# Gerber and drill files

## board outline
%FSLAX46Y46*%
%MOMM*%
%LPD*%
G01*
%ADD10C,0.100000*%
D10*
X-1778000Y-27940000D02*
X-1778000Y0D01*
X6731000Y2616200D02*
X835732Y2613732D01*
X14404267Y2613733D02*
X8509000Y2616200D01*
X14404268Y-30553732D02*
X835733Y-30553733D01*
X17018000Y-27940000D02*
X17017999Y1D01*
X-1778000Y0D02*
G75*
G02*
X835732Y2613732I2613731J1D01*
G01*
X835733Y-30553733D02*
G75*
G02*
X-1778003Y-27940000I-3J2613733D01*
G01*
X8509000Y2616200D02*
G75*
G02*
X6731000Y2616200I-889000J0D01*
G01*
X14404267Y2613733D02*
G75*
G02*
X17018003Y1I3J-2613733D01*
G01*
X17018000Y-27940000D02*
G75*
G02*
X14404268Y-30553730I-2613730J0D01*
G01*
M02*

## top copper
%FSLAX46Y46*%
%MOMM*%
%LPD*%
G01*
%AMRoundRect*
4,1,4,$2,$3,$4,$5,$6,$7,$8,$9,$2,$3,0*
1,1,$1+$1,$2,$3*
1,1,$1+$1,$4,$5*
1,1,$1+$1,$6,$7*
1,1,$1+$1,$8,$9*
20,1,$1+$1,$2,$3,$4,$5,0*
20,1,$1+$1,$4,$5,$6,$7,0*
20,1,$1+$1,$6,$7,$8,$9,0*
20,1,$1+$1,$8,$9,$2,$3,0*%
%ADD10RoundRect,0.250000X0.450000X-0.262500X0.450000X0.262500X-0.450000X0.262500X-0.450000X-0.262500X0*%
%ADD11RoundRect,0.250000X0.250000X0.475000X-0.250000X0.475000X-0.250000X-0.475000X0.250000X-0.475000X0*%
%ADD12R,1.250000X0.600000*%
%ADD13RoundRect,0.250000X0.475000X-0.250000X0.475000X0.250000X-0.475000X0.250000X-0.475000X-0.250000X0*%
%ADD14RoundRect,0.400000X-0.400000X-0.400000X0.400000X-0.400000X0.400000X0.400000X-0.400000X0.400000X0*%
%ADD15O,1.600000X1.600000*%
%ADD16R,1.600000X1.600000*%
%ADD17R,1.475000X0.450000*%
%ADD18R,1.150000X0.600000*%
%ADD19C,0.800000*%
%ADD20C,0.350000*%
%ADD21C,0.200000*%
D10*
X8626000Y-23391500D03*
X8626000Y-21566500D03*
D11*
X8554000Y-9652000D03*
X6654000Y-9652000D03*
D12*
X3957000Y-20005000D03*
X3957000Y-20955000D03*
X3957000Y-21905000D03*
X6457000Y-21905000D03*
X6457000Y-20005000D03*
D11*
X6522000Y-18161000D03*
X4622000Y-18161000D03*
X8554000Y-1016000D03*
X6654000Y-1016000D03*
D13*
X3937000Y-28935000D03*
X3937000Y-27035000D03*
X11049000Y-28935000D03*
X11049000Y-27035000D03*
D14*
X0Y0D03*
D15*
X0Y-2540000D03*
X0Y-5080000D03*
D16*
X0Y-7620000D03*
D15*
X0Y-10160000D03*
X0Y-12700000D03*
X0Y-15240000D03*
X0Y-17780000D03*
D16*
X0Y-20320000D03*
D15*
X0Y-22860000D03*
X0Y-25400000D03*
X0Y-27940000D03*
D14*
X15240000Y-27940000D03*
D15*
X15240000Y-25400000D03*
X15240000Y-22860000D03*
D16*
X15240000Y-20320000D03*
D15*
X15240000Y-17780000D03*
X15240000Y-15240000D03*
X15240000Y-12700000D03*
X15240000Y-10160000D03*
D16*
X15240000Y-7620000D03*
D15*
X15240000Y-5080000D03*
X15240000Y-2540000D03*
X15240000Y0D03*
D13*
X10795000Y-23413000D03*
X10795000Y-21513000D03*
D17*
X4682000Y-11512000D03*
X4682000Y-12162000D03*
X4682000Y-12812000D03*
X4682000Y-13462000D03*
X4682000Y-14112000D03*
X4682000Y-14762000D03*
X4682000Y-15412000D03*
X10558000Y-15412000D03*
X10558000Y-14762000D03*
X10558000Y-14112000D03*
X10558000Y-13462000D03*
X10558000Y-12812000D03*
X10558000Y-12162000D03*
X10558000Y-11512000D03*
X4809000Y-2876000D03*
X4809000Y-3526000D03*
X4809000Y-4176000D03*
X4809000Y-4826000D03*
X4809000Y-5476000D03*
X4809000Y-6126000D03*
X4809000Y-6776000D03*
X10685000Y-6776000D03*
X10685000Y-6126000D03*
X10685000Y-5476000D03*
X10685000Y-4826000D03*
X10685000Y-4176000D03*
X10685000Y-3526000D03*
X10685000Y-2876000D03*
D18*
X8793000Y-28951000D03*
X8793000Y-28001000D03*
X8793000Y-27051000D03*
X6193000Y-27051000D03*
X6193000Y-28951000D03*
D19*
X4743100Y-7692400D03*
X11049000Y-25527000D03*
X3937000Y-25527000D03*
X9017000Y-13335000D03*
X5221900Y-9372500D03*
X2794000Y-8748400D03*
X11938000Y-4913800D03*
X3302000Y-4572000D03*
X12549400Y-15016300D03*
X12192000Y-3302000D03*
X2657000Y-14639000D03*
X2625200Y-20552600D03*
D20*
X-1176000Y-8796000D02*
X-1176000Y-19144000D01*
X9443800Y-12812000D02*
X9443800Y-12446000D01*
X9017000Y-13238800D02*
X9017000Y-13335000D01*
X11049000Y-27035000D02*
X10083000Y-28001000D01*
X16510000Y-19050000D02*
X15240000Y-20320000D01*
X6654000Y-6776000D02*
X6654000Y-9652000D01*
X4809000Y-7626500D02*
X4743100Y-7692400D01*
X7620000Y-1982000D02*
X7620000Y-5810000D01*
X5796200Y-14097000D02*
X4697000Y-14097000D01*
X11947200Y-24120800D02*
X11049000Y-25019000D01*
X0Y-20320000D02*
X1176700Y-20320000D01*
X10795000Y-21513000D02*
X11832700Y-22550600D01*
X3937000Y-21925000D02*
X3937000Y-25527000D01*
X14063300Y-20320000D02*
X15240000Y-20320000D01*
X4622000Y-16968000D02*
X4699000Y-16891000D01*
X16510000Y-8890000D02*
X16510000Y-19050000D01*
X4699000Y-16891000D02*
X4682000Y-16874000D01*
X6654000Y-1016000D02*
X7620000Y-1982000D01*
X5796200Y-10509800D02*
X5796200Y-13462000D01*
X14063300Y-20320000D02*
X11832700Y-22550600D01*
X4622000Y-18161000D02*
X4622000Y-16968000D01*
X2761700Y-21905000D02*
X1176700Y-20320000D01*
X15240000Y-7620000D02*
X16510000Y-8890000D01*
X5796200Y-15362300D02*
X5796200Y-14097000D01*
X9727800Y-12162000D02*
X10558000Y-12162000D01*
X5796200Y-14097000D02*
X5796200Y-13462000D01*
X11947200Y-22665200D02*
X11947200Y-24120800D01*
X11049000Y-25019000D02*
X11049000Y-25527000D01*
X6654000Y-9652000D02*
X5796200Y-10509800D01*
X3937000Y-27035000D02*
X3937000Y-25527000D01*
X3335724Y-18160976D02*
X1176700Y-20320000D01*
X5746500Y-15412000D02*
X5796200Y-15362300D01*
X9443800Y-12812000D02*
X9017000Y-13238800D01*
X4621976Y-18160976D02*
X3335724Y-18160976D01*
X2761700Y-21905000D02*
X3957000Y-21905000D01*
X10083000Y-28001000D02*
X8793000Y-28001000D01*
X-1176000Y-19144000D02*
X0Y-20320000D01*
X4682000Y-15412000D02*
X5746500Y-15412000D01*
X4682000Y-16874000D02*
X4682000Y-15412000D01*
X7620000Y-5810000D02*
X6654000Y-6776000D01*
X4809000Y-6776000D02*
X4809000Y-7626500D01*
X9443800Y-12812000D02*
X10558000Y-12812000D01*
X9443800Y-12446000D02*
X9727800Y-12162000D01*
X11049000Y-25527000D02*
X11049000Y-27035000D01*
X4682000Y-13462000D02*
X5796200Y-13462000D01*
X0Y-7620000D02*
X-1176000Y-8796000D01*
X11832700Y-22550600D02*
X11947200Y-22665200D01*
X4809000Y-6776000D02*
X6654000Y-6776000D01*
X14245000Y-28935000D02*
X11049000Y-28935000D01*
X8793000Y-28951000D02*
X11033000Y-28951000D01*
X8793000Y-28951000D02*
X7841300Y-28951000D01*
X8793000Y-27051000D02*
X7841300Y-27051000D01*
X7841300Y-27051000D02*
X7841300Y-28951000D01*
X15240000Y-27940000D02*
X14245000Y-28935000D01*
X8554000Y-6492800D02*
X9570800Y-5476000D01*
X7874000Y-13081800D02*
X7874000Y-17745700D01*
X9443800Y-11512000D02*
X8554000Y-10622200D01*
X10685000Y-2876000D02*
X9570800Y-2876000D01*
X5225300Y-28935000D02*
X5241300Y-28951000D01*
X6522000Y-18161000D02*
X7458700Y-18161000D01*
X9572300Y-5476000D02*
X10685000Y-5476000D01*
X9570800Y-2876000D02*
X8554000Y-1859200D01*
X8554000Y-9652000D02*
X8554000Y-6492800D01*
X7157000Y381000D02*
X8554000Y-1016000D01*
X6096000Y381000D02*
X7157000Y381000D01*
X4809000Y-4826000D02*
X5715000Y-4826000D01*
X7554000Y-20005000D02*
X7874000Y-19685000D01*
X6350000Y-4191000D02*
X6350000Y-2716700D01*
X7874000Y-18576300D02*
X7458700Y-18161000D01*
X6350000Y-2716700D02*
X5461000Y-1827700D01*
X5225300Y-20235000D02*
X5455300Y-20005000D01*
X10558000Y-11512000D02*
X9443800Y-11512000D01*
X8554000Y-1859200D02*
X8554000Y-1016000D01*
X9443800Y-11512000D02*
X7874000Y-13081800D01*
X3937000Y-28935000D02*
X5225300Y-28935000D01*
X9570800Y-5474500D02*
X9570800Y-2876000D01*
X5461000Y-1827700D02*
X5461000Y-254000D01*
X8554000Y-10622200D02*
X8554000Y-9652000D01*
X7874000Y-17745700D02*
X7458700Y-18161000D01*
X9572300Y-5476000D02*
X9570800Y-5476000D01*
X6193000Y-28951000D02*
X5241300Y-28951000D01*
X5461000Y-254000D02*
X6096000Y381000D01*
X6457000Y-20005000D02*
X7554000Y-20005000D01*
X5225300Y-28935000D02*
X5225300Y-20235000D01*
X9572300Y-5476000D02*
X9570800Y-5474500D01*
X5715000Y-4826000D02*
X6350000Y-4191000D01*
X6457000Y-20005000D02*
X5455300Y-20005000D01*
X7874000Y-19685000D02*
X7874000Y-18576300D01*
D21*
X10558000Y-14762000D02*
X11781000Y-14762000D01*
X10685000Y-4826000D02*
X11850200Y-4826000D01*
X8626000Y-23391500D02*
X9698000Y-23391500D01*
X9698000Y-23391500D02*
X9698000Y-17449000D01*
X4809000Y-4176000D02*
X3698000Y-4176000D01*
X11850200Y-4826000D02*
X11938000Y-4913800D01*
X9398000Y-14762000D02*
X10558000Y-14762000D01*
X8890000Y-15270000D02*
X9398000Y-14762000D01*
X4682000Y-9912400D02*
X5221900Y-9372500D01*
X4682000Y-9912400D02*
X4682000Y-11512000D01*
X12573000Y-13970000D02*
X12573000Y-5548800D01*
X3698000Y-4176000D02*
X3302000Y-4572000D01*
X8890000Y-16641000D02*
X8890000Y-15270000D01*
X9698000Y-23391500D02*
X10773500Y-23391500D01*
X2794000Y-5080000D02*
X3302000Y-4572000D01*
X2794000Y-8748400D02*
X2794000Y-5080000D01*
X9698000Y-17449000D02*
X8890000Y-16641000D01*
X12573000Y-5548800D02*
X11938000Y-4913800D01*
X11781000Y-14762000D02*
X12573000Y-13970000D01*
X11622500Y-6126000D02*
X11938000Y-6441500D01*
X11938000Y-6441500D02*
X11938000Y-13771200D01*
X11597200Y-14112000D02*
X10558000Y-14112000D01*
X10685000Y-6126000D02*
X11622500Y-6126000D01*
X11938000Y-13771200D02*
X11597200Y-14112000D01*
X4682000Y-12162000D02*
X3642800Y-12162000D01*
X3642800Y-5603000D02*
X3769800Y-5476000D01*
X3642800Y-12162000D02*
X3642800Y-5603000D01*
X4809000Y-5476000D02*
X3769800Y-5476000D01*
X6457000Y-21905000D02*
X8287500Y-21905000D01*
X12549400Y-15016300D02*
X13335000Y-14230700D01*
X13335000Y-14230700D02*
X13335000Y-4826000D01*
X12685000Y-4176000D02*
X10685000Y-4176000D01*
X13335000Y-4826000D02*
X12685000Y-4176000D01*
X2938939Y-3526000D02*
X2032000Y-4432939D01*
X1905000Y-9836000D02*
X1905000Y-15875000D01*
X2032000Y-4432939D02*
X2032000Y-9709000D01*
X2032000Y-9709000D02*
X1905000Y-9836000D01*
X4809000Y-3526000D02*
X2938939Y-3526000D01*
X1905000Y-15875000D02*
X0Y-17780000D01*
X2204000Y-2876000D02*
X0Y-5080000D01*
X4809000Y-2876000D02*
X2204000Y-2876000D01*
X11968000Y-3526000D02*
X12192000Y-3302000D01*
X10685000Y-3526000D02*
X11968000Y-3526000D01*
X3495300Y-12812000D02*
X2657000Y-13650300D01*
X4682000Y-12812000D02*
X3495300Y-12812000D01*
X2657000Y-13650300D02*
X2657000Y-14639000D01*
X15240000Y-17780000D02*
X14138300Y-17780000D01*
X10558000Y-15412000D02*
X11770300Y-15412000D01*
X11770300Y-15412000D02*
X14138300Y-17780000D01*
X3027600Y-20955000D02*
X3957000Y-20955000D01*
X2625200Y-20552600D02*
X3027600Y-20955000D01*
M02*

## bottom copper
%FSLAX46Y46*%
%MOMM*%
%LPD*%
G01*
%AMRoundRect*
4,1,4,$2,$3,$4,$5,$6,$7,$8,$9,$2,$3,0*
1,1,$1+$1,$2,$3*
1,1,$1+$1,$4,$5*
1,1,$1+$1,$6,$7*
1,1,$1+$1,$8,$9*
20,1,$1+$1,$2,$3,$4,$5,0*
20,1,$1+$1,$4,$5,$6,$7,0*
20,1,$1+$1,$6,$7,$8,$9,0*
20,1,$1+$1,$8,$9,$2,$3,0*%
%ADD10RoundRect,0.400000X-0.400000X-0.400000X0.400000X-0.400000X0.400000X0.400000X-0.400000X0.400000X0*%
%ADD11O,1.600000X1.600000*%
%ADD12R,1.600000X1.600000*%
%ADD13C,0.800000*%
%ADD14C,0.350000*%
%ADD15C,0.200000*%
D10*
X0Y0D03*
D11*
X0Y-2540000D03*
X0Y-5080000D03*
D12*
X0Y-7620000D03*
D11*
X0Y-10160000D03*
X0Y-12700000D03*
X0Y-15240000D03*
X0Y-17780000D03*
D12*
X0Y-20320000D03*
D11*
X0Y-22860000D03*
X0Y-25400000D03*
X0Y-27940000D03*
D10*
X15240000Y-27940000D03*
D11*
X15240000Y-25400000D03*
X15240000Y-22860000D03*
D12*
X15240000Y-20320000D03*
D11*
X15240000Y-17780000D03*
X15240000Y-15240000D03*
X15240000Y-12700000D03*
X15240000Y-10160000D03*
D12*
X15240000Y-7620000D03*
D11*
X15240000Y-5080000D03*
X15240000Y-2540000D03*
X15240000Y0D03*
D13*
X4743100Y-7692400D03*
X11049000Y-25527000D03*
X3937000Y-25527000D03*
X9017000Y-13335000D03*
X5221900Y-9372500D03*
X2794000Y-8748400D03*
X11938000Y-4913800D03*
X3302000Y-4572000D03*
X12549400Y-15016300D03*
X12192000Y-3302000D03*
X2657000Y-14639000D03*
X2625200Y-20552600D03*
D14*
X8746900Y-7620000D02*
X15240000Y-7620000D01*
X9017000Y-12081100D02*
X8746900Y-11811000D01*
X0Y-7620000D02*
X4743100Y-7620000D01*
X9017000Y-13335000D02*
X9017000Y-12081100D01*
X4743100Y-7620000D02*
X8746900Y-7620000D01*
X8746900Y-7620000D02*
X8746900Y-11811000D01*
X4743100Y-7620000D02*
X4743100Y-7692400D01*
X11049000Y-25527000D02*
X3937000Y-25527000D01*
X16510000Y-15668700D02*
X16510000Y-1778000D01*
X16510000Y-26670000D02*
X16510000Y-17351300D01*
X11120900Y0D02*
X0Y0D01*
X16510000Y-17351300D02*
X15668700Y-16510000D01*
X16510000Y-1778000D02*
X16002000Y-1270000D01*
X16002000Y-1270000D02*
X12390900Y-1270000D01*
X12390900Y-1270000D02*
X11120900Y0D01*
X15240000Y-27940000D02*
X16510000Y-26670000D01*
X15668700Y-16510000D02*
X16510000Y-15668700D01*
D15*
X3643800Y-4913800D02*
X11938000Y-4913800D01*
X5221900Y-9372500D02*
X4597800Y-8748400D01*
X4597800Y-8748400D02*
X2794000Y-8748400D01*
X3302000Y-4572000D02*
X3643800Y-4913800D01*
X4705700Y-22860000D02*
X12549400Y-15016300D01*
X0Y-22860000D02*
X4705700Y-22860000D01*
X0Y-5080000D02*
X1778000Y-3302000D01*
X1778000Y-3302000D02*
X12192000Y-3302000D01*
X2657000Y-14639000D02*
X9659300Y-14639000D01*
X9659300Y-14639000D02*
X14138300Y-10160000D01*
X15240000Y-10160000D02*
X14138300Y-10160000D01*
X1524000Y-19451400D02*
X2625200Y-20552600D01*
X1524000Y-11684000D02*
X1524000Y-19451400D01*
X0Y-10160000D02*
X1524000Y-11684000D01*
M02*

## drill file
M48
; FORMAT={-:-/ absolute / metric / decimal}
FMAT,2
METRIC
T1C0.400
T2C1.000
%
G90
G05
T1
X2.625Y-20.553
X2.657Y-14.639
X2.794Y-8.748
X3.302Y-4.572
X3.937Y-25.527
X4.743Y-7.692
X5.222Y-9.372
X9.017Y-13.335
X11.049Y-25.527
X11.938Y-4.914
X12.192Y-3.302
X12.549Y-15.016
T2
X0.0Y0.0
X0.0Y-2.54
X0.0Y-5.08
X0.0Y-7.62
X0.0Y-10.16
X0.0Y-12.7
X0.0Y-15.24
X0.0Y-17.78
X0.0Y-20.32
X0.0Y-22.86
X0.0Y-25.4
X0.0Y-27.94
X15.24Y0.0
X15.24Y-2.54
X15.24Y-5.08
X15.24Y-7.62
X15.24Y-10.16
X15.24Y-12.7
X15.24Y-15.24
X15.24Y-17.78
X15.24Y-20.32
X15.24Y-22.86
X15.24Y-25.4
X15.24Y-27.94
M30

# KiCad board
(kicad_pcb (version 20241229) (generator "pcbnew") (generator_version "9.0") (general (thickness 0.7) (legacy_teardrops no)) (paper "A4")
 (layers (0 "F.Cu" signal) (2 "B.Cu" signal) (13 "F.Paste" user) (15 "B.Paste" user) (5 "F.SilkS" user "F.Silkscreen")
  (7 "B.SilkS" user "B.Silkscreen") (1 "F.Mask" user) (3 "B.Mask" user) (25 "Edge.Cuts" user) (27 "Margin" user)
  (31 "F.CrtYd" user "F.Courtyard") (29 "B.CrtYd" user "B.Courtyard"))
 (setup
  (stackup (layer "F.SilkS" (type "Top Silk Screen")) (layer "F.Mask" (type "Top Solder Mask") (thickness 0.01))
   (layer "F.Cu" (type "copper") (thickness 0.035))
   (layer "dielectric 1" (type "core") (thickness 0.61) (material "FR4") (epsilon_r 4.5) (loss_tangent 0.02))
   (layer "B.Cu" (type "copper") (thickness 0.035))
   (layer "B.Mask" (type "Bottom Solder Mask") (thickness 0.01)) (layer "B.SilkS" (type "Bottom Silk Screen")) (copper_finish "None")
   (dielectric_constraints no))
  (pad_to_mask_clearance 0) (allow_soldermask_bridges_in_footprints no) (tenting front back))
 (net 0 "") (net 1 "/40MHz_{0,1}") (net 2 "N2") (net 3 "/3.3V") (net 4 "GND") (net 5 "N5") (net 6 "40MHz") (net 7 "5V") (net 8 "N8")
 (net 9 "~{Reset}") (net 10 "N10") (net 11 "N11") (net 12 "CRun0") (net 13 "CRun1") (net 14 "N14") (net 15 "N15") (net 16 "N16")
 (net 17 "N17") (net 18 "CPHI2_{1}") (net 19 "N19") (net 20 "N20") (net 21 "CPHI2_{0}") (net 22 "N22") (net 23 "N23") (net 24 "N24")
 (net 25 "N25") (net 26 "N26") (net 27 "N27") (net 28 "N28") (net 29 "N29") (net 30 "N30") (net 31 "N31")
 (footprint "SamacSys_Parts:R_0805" (layer "F.Cu") (at 8.636 22.479)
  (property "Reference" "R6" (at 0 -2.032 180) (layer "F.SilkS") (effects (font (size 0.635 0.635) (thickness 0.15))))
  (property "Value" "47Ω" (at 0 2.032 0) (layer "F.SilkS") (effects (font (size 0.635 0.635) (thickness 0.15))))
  (pad "1" smd roundrect (at -0.01 0.9125 90) (size 1.025 1.4) (layers "F.Cu" "F.Mask" "F.Paste") (roundrect_rratio 0.243902)
   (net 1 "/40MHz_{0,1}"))
  (pad "2" smd roundrect (at -0.01 -0.9125 90) (size 1.025 1.4) (layers "F.Cu" "F.Mask" "F.Paste") (roundrect_rratio 0.243902) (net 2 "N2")))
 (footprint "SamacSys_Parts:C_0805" (layer "F.Cu") (at 7.62 9.652 90)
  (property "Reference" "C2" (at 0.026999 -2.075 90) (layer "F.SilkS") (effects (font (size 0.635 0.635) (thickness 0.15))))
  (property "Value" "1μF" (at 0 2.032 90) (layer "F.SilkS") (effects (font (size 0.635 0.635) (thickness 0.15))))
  (pad "1" smd roundrect (at 0 0.934 180) (size 1 1.45) (layers "F.Cu" "F.Mask" "F.Paste") (roundrect_rratio 0.25) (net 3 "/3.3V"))
  (pad "2" smd roundrect (at 0 -0.966 180) (size 1 1.45) (layers "F.Cu" "F.Mask" "F.Paste") (roundrect_rratio 0.25) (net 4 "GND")))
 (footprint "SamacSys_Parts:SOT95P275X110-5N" (layer "F.Cu") (at 5.207 20.955)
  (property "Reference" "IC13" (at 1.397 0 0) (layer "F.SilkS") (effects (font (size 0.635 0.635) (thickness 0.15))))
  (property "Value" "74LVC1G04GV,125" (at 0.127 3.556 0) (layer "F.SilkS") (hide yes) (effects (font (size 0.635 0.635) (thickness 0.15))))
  (pad "1" smd rect (at -1.25 -0.95 90) (size 0.6 1.25) (layers "F.Cu" "F.Mask" "F.Paste") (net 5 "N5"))
  (pad "2" smd rect (at -1.25 0 90) (size 0.6 1.25) (layers "F.Cu" "F.Mask" "F.Paste") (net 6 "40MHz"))
  (pad "3" smd rect (at -1.25 0.95 90) (size 0.6 1.25) (layers "F.Cu" "F.Mask" "F.Paste") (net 4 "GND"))
  (pad "4" smd rect (at 1.25 0.95 90) (size 0.6 1.25) (layers "F.Cu" "F.Mask" "F.Paste") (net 2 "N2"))
  (pad "5" smd rect (at 1.25 -0.95 90) (size 0.6 1.25) (layers "F.Cu" "F.Mask" "F.Paste") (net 3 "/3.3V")))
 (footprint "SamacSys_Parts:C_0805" (layer "F.Cu") (at 5.588 18.161 90)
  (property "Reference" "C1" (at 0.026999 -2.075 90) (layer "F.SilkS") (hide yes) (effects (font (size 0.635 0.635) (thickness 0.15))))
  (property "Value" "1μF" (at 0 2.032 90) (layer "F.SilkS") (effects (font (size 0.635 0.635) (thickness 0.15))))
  (pad "1" smd roundrect (at 0 0.934 180) (size 1 1.45) (layers "F.Cu" "F.Mask" "F.Paste") (roundrect_rratio 0.25) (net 3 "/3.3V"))
  (pad "2" smd roundrect (at 0 -0.966 180) (size 1 1.45) (layers "F.Cu" "F.Mask" "F.Paste") (roundrect_rratio 0.25) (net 4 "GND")))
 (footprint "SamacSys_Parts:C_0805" (layer "F.Cu") (at 7.62 1.016 90)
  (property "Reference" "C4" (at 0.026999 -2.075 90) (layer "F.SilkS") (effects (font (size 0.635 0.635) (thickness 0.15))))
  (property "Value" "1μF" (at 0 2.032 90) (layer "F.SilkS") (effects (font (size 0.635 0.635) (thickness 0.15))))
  (pad "1" smd roundrect (at 0 0.934 180) (size 1 1.45) (layers "F.Cu" "F.Mask" "F.Paste") (roundrect_rratio 0.25) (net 3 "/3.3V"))
  (pad "2" smd roundrect (at 0 -0.966 180) (size 1 1.45) (layers "F.Cu" "F.Mask" "F.Paste") (roundrect_rratio 0.25) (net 4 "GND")))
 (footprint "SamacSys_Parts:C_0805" (layer "F.Cu") (at 3.937 28.001)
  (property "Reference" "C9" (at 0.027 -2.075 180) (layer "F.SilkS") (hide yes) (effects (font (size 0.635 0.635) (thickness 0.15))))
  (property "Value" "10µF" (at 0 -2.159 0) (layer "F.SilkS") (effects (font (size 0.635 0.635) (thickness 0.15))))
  (pad "1" smd roundrect (at 0 0.934 90) (size 1 1.45) (layers "F.Cu" "F.Mask" "F.Paste") (roundrect_rratio 0.25) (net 3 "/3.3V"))
  (pad "2" smd roundrect (at 0 -0.966 90) (size 1 1.45) (layers "F.Cu" "F.Mask" "F.Paste") (roundrect_rratio 0.25) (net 4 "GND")))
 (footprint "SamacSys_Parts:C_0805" (layer "F.Cu") (at 11.049 28.001)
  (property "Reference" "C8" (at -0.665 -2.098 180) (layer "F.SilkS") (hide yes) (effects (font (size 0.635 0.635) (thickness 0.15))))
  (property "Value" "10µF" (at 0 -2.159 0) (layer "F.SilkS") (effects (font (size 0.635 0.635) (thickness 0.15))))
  (pad "1" smd roundrect (at 0 0.934 90) (size 1 1.45) (layers "F.Cu" "F.Mask" "F.Paste") (roundrect_rratio 0.25) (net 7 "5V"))
  (pad "2" smd roundrect (at 0 -0.966 90) (size 1 1.45) (layers "F.Cu" "F.Mask" "F.Paste") (roundrect_rratio 0.25) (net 4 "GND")))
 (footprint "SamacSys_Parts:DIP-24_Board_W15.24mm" (layer "F.Cu") (at 0 0)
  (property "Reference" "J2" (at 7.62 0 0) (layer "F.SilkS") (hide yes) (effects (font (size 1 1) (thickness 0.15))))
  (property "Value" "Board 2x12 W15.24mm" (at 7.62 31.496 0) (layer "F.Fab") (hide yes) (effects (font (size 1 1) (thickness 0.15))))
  (fp_line (start -1.778 27.94) (end -1.778 0) (stroke (width 0.1) (type solid)) (layer "Edge.Cuts"))
  (fp_line (start 6.731 -2.6162) (end 0.835732 -2.613732) (stroke (width 0.1) (type solid)) (layer "Edge.Cuts"))
  (fp_line (start 14.404267 -2.613733) (end 8.509 -2.6162) (stroke (width 0.1) (type solid)) (layer "Edge.Cuts"))
  (fp_line (start 14.404268 30.553732) (end 0.835733 30.553733) (stroke (width 0.1) (type solid)) (layer "Edge.Cuts"))
  (fp_line (start 17.018 27.94) (end 17.017999 -0.000001) (stroke (width 0.1) (type solid)) (layer "Edge.Cuts"))
  (fp_arc (start -1.778 0) (mid -1.012456 -1.848188) (end 0.835732 -2.613732) (stroke (width 0.1) (type solid)) (layer "Edge.Cuts"))
  (fp_arc (start 0.835733 30.553733) (mid -1.012456 29.788189) (end -1.778 27.94) (stroke (width 0.1) (type solid)) (layer "Edge.Cuts"))
  (fp_arc (start 8.509 -2.6162) (mid 7.62 -1.7272) (end 6.731 -2.6162) (stroke (width 0.1) (type default)) (layer "Edge.Cuts"))
  (fp_arc (start 14.404267 -2.613733) (mid 16.252455 -1.848189) (end 17.017999 -0.000001) (stroke (width 0.1) (type solid))
   (layer "Edge.Cuts"))
  (fp_arc (start 17.018 27.94) (mid 16.252455 29.788187) (end 14.404268 30.553732) (stroke (width 0.1) (type solid)) (layer "Edge.Cuts"))
  (pad "1" thru_hole roundrect (at 0 0) (size 1.6 1.6) (drill 1) (layers "*.Cu" "*.Mask") (remove_unused_layers no) (roundrect_rratio 0.25)
   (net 7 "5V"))
  (pad "2" thru_hole oval (at 0 2.54) (size 1.6 1.6) (drill 1) (layers "*.Cu" "*.Mask") (remove_unused_layers no) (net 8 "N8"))
  (pad "3" thru_hole oval (at 0 5.08) (size 1.6 1.6) (drill 1) (layers "*.Cu" "*.Mask") (remove_unused_layers no) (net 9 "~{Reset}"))
  (pad "4" thru_hole rect (at 0 7.62) (size 1.6 1.6) (drill 1) (layers "*.Cu" "*.Mask") (remove_unused_layers no) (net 4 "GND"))
  (pad "5" thru_hole oval (at 0 10.16) (size 1.6 1.6) (drill 1) (layers "*.Cu" "*.Mask") (remove_unused_layers no) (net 6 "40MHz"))
  (pad "6" thru_hole oval (at 0 12.7) (size 1.6 1.6) (drill 1) (layers "*.Cu" "*.Mask") (remove_unused_layers no) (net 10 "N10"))
  (pad "7" thru_hole oval (at 0 15.24) (size 1.6 1.6) (drill 1) (layers "*.Cu" "*.Mask") (remove_unused_layers no) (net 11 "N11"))
  (pad "8" thru_hole oval (at 0 17.78) (size 1.6 1.6) (drill 1) (layers "*.Cu" "*.Mask") (remove_unused_layers no) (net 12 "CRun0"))
  (pad "9" thru_hole rect (at 0 20.32) (size 1.6 1.6) (drill 1) (layers "*.Cu" "*.Mask") (remove_unused_layers no) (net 4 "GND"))
  (pad "10" thru_hole oval (at 0 22.86) (size 1.6 1.6) (drill 1) (layers "*.Cu" "*.Mask") (remove_unused_layers no) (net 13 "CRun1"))
  (pad "11" thru_hole oval (at 0 25.4) (size 1.6 1.6) (drill 1) (layers "*.Cu" "*.Mask") (remove_unused_layers no) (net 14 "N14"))
  (pad "12" thru_hole oval (at 0 27.94) (size 1.6 1.6) (drill 1) (layers "*.Cu" "*.Mask") (remove_unused_layers no) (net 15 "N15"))
  (pad "13" thru_hole roundrect (at 15.24 27.94) (size 1.6 1.6) (drill 1) (layers "*.Cu" "*.Mask") (remove_unused_layers no)
   (roundrect_rratio 0.25) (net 7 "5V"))
  (pad "14" thru_hole oval (at 15.24 25.4) (size 1.6 1.6) (drill 1) (layers "*.Cu" "*.Mask") (remove_unused_layers no) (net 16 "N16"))
  (pad "15" thru_hole oval (at 15.24 22.86) (size 1.6 1.6) (drill 1) (layers "*.Cu" "*.Mask") (remove_unused_layers no) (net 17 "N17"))
  (pad "16" thru_hole rect (at 15.24 20.32) (size 1.6 1.6) (drill 1) (layers "*.Cu" "*.Mask") (remove_unused_layers no) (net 4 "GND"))
  (pad "17" thru_hole oval (at 15.24 17.78 180) (size 1.6 1.6) (drill 1) (layers "*.Cu" "*.Mask") (remove_unused_layers no)
   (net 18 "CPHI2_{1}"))
  (pad "18" thru_hole oval (at 15.24 15.24 180) (size 1.6 1.6) (drill 1) (layers "*.Cu" "*.Mask") (remove_unused_layers no) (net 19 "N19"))
  (pad "19" thru_hole oval (at 15.24 12.7 180) (size 1.6 1.6) (drill 1) (layers "*.Cu" "*.Mask") (remove_unused_layers no) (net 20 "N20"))
  (pad "20" thru_hole oval (at 15.24 10.16 180) (size 1.6 1.6) (drill 1) (layers "*.Cu" "*.Mask") (remove_unused_layers no)
   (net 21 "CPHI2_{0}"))
  (pad "21" thru_hole rect (at 15.24 7.62) (size 1.6 1.6) (drill 1) (layers "*.Cu" "*.Mask") (remove_unused_layers no) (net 4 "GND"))
  (pad "22" thru_hole oval (at 15.24 5.08) (size 1.6 1.6) (drill 1) (layers "*.Cu" "*.Mask") (remove_unused_layers no) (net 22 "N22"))
  (pad "23" thru_hole oval (at 15.24 2.54) (size 1.6 1.6) (drill 1) (layers "*.Cu" "*.Mask") (remove_unused_layers no) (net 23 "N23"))
  (pad "24" thru_hole oval (at 15.24 0) (size 1.6 1.6) (drill 1) (layers "*.Cu" "*.Mask") (remove_unused_layers no) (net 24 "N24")))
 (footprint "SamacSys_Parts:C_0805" (layer "F.Cu") (at 10.795 22.479)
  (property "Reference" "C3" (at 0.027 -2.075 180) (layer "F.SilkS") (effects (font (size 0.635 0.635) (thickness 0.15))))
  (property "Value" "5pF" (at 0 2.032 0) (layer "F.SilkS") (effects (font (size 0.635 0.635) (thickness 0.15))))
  (pad "1" smd roundrect (at 0 0.934 90) (size 1 1.45) (layers "F.Cu" "F.Mask" "F.Paste") (roundrect_rratio 0.25) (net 1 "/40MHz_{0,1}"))
  (pad "2" smd roundrect (at 0 -0.966 90) (size 1 1.45) (layers "F.Cu" "F.Mask" "F.Paste") (roundrect_rratio 0.25) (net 4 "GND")))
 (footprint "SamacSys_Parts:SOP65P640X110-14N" (layer "F.Cu") (at 7.62 13.462)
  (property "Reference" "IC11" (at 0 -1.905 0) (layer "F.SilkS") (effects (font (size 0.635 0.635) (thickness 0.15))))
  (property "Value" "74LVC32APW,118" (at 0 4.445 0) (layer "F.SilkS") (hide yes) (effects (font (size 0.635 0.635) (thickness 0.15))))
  (pad "1" smd rect (at -2.938 -1.95 90) (size 0.45 1.475) (layers "F.Cu" "F.Mask" "F.Paste") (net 1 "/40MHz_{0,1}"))
  (pad "2" smd rect (at -2.938 -1.3 90) (size 0.45 1.475) (layers "F.Cu" "F.Mask" "F.Paste") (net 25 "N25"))
  (pad "3" smd rect (at -2.938 -0.65 90) (size 0.45 1.475) (layers "F.Cu" "F.Mask" "F.Paste") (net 21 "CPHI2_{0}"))
  (pad "4" smd rect (at -2.938 0 90) (size 0.45 1.475) (layers "F.Cu" "F.Mask" "F.Paste") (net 4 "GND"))
  (pad "5" smd rect (at -2.938 0.65 90) (size 0.45 1.475) (layers "F.Cu" "F.Mask" "F.Paste") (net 4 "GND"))
  (pad "6" smd rect (at -2.938 1.3 90) (size 0.45 1.475) (layers "F.Cu" "F.Mask" "F.Paste") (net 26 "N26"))
  (pad "7" smd rect (at -2.938 1.95 90) (size 0.45 1.475) (layers "F.Cu" "F.Mask" "F.Paste") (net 4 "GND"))
  (pad "8" smd rect (at 2.938 1.95 90) (size 0.45 1.475) (layers "F.Cu" "F.Mask" "F.Paste") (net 18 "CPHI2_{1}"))
  (pad "9" smd rect (at 2.938 1.3 90) (size 0.45 1.475) (layers "F.Cu" "F.Mask" "F.Paste") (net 1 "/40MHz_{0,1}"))
  (pad "10" smd rect (at 2.938 0.65 90) (size 0.45 1.475) (layers "F.Cu" "F.Mask" "F.Paste") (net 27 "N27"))
  (pad "11" smd rect (at 2.938 0 90) (size 0.45 1.475) (layers "F.Cu" "F.Mask" "F.Paste") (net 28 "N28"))
  (pad "12" smd rect (at 2.938 -0.65 90) (size 0.45 1.475) (layers "F.Cu" "F.Mask" "F.Paste") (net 4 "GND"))
  (pad "13" smd rect (at 2.938 -1.3 90) (size 0.45 1.475) (layers "F.Cu" "F.Mask" "F.Paste") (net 4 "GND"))
  (pad "14" smd rect (at 2.938 -1.95 90) (size 0.45 1.475) (layers "F.Cu" "F.Mask" "F.Paste") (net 3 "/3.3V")))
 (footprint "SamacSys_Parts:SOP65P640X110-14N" (layer "F.Cu") (at 7.747 4.826)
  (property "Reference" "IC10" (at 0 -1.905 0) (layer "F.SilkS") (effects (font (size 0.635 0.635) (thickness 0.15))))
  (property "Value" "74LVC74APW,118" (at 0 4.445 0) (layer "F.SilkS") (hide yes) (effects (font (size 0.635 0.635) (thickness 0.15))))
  (pad "1" smd rect (at -2.938 -1.95 90) (size 0.45 1.475) (layers "F.Cu" "F.Mask" "F.Paste") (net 9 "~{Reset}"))
  (pad "2" smd rect (at -2.938 -1.3 90) (size 0.45 1.475) (layers "F.Cu" "F.Mask" "F.Paste") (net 12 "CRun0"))
  (pad "3" smd rect (at -2.938 -0.65 90) (size 0.45 1.475) (layers "F.Cu" "F.Mask" "F.Paste") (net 1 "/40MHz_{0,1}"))
  (pad "4" smd rect (at -2.938 0 90) (size 0.45 1.475) (layers "F.Cu" "F.Mask" "F.Paste") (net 3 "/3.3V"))
  (pad "5" smd rect (at -2.938 0.65 90) (size 0.45 1.475) (layers "F.Cu" "F.Mask" "F.Paste") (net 25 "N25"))
  (pad "6" smd rect (at -2.938 1.3 90) (size 0.45 1.475) (layers "F.Cu" "F.Mask" "F.Paste") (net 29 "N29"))
  (pad "7" smd rect (at -2.938 1.95 90) (size 0.45 1.475) (layers "F.Cu" "F.Mask" "F.Paste") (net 4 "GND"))
  (pad "8" smd rect (at 2.938 1.95 90) (size 0.45 1.475) (layers "F.Cu" "F.Mask" "F.Paste") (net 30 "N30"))
  (pad "9" smd rect (at 2.938 1.3 90) (size 0.45 1.475) (layers "F.Cu" "F.Mask" "F.Paste") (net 27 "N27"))
  (pad "10" smd rect (at 2.938 0.65 90) (size 0.45 1.475) (layers "F.Cu" "F.Mask" "F.Paste") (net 3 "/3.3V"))
  (pad "11" smd rect (at 2.938 0 90) (size 0.45 1.475) (layers "F.Cu" "F.Mask" "F.Paste") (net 1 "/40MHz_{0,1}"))
  (pad "12" smd rect (at 2.938 -0.65 90) (size 0.45 1.475) (layers "F.Cu" "F.Mask" "F.Paste") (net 13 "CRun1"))
  (pad "13" smd rect (at 2.938 -1.3 90) (size 0.45 1.475) (layers "F.Cu" "F.Mask" "F.Paste") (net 9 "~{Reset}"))
  (pad "14" smd rect (at 2.938 -1.95 90) (size 0.45 1.475) (layers "F.Cu" "F.Mask" "F.Paste") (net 3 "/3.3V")))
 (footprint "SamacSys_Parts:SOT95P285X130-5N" (layer "F.Cu") (at 7.493 28.001 180)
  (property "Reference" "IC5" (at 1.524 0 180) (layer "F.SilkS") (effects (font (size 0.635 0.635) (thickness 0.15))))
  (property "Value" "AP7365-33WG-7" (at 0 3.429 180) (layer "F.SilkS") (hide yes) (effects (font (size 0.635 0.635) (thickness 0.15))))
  (pad "1" smd rect (at -1.3 -0.95 270) (size 0.6 1.15) (layers "F.Cu" "F.Mask" "F.Paste") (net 7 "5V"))
  (pad "2" smd rect (at -1.3 0 270) (size 0.6 1.15) (layers "F.Cu" "F.Mask" "F.Paste") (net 4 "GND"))
  (pad "3" smd rect (at -1.3 0.95 270) (size 0.6 1.15) (layers "F.Cu" "F.Mask" "F.Paste") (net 7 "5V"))
  (pad "4" smd rect (at 1.3 0.95 270) (size 0.6 1.15) (layers "F.Cu" "F.Mask" "F.Paste") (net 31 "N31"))
  (pad "5" smd rect (at 1.3 -0.95 270) (size 0.6 1.15) (layers "F.Cu" "F.Mask" "F.Paste") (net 3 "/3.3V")))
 (segment (start -1.176 8.796) (end -1.176 19.144) (width 0.35) (layer "F.Cu") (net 4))
 (segment (start 9.4438 12.812) (end 9.4438 12.446) (width 0.35) (layer "F.Cu") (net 4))
 (segment (start 9.017 13.2388) (end 9.017 13.335) (width 0.35) (layer "F.Cu") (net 4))
 (segment (start 11.049 27.035) (end 10.083 28.001) (width 0.35) (layer "F.Cu") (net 4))
 (segment (start 16.51 19.05) (end 15.24 20.32) (width 0.35) (layer "F.Cu") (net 4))
 (segment (start 6.654 6.776) (end 6.654 9.652) (width 0.35) (layer "F.Cu") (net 4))
 (segment (start 4.809 7.6265) (end 4.7431 7.6924) (width 0.35) (layer "F.Cu") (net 4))
 (segment (start 7.62 1.982) (end 7.62 5.81) (width 0.35) (layer "F.Cu") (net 4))
 (segment (start 5.7962 14.097) (end 4.697 14.097) (width 0.35) (layer "F.Cu") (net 4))
 (segment (start 11.9472 24.1208) (end 11.049 25.019) (width 0.35) (layer "F.Cu") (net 4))
 (segment (start 0 20.32) (end 1.1767 20.32) (width 0.35) (layer "F.Cu") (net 4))
 (segment (start 10.795 21.513) (end 11.8327 22.5506) (width 0.35) (layer "F.Cu") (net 4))
 (segment (start 3.937 21.925) (end 3.937 25.527) (width 0.35) (layer "F.Cu") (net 4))
 (segment (start 14.0633 20.32) (end 15.24 20.32) (width 0.35) (layer "F.Cu") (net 4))
 (segment (start 4.622 16.968) (end 4.699 16.891) (width 0.35) (layer "F.Cu") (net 4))
 (segment (start 16.51 8.89) (end 16.51 19.05) (width 0.35) (layer "F.Cu") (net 4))
 (segment (start 4.699 16.891) (end 4.682 16.874) (width 0.35) (layer "F.Cu") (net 4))
 (segment (start 6.654 1.016) (end 7.62 1.982) (width 0.35) (layer "F.Cu") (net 4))
 (segment (start 5.7962 10.5098) (end 5.7962 13.462) (width 0.35) (layer "F.Cu") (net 4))
 (segment (start 14.0633 20.32) (end 11.8327 22.5506) (width 0.35) (layer "F.Cu") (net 4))
 (segment (start 4.622 18.161) (end 4.622 16.968) (width 0.35) (layer "F.Cu") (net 4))
 (segment (start 2.7617 21.905) (end 1.1767 20.32) (width 0.35) (layer "F.Cu") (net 4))
 (segment (start 15.24 7.62) (end 16.51 8.89) (width 0.35) (layer "F.Cu") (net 4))
 (segment (start 5.7962 15.3623) (end 5.7962 14.097) (width 0.35) (layer "F.Cu") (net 4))
 (segment (start 9.7278 12.162) (end 10.558 12.162) (width 0.35) (layer "F.Cu") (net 4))
 (segment (start 5.7962 14.097) (end 5.7962 13.462) (width 0.35) (layer "F.Cu") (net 4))
 (segment (start 11.9472 22.6652) (end 11.9472 24.1208) (width 0.35) (layer "F.Cu") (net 4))
 (segment (start 11.049 25.019) (end 11.049 25.527) (width 0.35) (layer "F.Cu") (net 4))
 (segment (start 6.654 9.652) (end 5.7962 10.5098) (width 0.35) (layer "F.Cu") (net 4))
 (segment (start 3.937 27.035) (end 3.937 25.527) (width 0.35) (layer "F.Cu") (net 4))
 (segment (start 3.335724 18.160976) (end 1.1767 20.32) (width 0.35) (layer "F.Cu") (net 4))
 (segment (start 5.7465 15.412) (end 5.7962 15.3623) (width 0.35) (layer "F.Cu") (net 4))
 (segment (start 9.4438 12.812) (end 9.017 13.2388) (width 0.35) (layer "F.Cu") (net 4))
 (segment (start 4.621976 18.160976) (end 3.335724 18.160976) (width 0.35) (layer "F.Cu") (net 4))
 (segment (start 2.7617 21.905) (end 3.957 21.905) (width 0.35) (layer "F.Cu") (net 4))
 (segment (start 10.083 28.001) (end 8.793 28.001) (width 0.35) (layer "F.Cu") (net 4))
 (segment (start -1.176 19.144) (end 0 20.32) (width 0.35) (layer "F.Cu") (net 4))
 (segment (start 4.682 15.412) (end 5.7465 15.412) (width 0.35) (layer "F.Cu") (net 4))
 (segment (start 4.682 16.874) (end 4.682 15.412) (width 0.35) (layer "F.Cu") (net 4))
 (segment (start 7.62 5.81) (end 6.654 6.776) (width 0.35) (layer "F.Cu") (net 4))
 (segment (start 4.809 6.776) (end 4.809 7.6265) (width 0.35) (layer "F.Cu") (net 4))
 (segment (start 9.4438 12.812) (end 10.558 12.812) (width 0.35) (layer "F.Cu") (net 4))
 (segment (start 9.4438 12.446) (end 9.7278 12.162) (width 0.35) (layer "F.Cu") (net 4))
 (segment (start 11.049 25.527) (end 11.049 27.035) (width 0.35) (layer "F.Cu") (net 4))
 (segment (start 4.682 13.462) (end 5.7962 13.462) (width 0.35) (layer "F.Cu") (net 4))
 (segment (start 0 7.62) (end -1.176 8.796) (width 0.35) (layer "F.Cu") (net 4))
 (segment (start 11.8327 22.5506) (end 11.9472 22.6652) (width 0.35) (layer "F.Cu") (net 4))
 (segment (start 4.809 6.776) (end 6.654 6.776) (width 0.35) (layer "F.Cu") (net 4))
 (via (at 4.7431 7.6924) (size 0.8) (drill 0.4) (layers "F.Cu" "B.Cu") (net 4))
 (via (at 11.049 25.527) (size 0.8) (drill 0.4) (layers "F.Cu" "B.Cu") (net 4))
 (via (at 3.937 25.527) (size 0.8) (drill 0.4) (layers "F.Cu" "B.Cu") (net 4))
 (via (at 9.017 13.335) (size 0.8) (drill 0.4) (layers "F.Cu" "B.Cu") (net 4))
 (segment (start 8.7469 7.62) (end 15.24 7.62) (width 0.35) (layer "B.Cu") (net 4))
 (segment (start 9.017 12.0811) (end 8.7469 11.811) (width 0.35) (layer "B.Cu") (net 4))
 (segment (start 0 7.62) (end 4.7431 7.62) (width 0.35) (layer "B.Cu") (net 4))
 (segment (start 9.017 13.335) (end 9.017 12.0811) (width 0.35) (layer "B.Cu") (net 4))
 (segment (start 4.7431 7.62) (end 8.7469 7.62) (width 0.35) (layer "B.Cu") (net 4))
 (segment (start 8.7469 7.62) (end 8.7469 11.811) (width 0.35) (layer "B.Cu") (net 4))
 (segment (start 4.7431 7.62) (end 4.7431 7.6924) (width 0.35) (layer "B.Cu") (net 4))
 (segment (start 11.049 25.527) (end 3.937 25.527) (width 0.35) (layer "B.Cu") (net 4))
 (segment (start 14.245 28.935) (end 11.049 28.935) (width 0.35) (layer "F.Cu") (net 7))
 (segment (start 8.793 28.951) (end 11.033 28.951) (width 0.35) (layer "F.Cu") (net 7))
 (segment (start 8.793 28.951) (end 7.8413 28.951) (width 0.35) (layer "F.Cu") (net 7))
 (segment (start 8.793 27.051) (end 7.8413 27.051) (width 0.35) (layer "F.Cu") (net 7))
 (segment (start 7.8413 27.051) (end 7.8413 28.951) (width 0.35) (layer "F.Cu") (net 7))
 (segment (start 15.24 27.94) (end 14.245 28.935) (width 0.35) (layer "F.Cu") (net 7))
 (segment (start 16.51 15.6687) (end 16.51 1.778) (width 0.35) (layer "B.Cu") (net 7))
 (segment (start 16.51 26.67) (end 16.51 17.3513) (width 0.35) (layer "B.Cu") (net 7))
 (segment (start 11.1209 0) (end 0 0) (width 0.35) (layer "B.Cu") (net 7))
 (segment (start 16.51 17.3513) (end 15.6687 16.51) (width 0.35) (layer "B.Cu") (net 7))
 (segment (start 16.51 1.778) (end 16.002 1.27) (width 0.35) (layer "B.Cu") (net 7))
 (segment (start 16.002 1.27) (end 12.3909 1.27) (width 0.35) (layer "B.Cu") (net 7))
 (segment (start 12.3909 1.27) (end 11.1209 0) (width 0.35) (layer "B.Cu") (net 7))
 (segment (start 15.24 27.94) (end 16.51 26.67) (width 0.35) (layer "B.Cu") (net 7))
 (segment (start 15.6687 16.51) (end 16.51 15.6687) (width 0.35) (layer "B.Cu") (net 7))
 (segment (start 8.554 6.4928) (end 9.5708 5.476) (width 0.35) (layer "F.Cu") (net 3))
 (segment (start 7.874 13.0818) (end 7.874 17.7457) (width 0.35) (layer "F.Cu") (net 3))
 (segment (start 9.4438 11.512) (end 8.554 10.6222) (width 0.35) (layer "F.Cu") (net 3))
 (segment (start 10.685 2.876) (end 9.5708 2.876) (width 0.35) (layer "F.Cu") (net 3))
 (segment (start 5.2253 28.935) (end 5.2413 28.951) (width 0.35) (layer "F.Cu") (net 3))
 (segment (start 6.522 18.161) (end 7.4587 18.161) (width 0.35) (layer "F.Cu") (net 3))
 (segment (start 9.5723 5.476) (end 10.685 5.476) (width 0.35) (layer "F.Cu") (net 3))
 (segment (start 9.5708 2.876) (end 8.554 1.8592) (width 0.35) (layer "F.Cu") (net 3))
 (segment (start 8.554 9.652) (end 8.554 6.4928) (width 0.35) (layer "F.Cu") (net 3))
 (segment (start 7.157 -0.381) (end 8.554 1.016) (width 0.35) (layer "F.Cu") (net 3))
 (segment (start 6.096 -0.381) (end 7.157 -0.381) (width 0.35) (layer "F.Cu") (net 3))
 (segment (start 4.809 4.826) (end 5.715 4.826) (width 0.35) (layer "F.Cu") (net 3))
 (segment (start 7.554 20.005) (end 7.874 19.685) (width 0.35) (layer "F.Cu") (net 3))
 (segment (start 6.35 4.191) (end 6.35 2.7167) (width 0.35) (layer "F.Cu") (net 3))
 (segment (start 7.874 18.5763) (end 7.4587 18.161) (width 0.35) (layer "F.Cu") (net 3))
 (segment (start 6.35 2.7167) (end 5.461 1.8277) (width 0.35) (layer "F.Cu") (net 3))
 (segment (start 5.2253 20.235) (end 5.4553 20.005) (width 0.35) (layer "F.Cu") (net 3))
 (segment (start 10.558 11.512) (end 9.4438 11.512) (width 0.35) (layer "F.Cu") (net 3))
 (segment (start 8.554 1.8592) (end 8.554 1.016) (width 0.35) (layer "F.Cu") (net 3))
 (segment (start 9.4438 11.512) (end 7.874 13.0818) (width 0.35) (layer "F.Cu") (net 3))
 (segment (start 3.937 28.935) (end 5.2253 28.935) (width 0.35) (layer "F.Cu") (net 3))
 (segment (start 9.5708 5.4745) (end 9.5708 2.876) (width 0.35) (layer "F.Cu") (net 3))
 (segment (start 5.461 1.8277) (end 5.461 0.254) (width 0.35) (layer "F.Cu") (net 3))
 (segment (start 8.554 10.6222) (end 8.554 9.652) (width 0.35) (layer "F.Cu") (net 3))
 (segment (start 7.874 17.7457) (end 7.4587 18.161) (width 0.35) (layer "F.Cu") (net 3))
 (segment (start 9.5723 5.476) (end 9.5708 5.476) (width 0.35) (layer "F.Cu") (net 3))
 (segment (start 6.193 28.951) (end 5.2413 28.951) (width 0.35) (layer "F.Cu") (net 3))
 (segment (start 5.461 0.254) (end 6.096 -0.381) (width 0.35) (layer "F.Cu") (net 3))
 (segment (start 6.457 20.005) (end 7.554 20.005) (width 0.35) (layer "F.Cu") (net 3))
 (segment (start 5.2253 28.935) (end 5.2253 20.235) (width 0.35) (layer "F.Cu") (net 3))
 (segment (start 9.5723 5.476) (end 9.5708 5.4745) (width 0.35) (layer "F.Cu") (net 3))
 (segment (start 5.715 4.826) (end 6.35 4.191) (width 0.35) (layer "F.Cu") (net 3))
 (segment (start 6.457 20.005) (end 5.4553 20.005) (width 0.35) (layer "F.Cu") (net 3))
 (segment (start 7.874 19.685) (end 7.874 18.5763) (width 0.35) (layer "F.Cu") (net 3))
 (segment (start 10.558 14.762) (end 11.781 14.762) (width 0.2) (layer "F.Cu") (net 1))
 (segment (start 10.685 4.826) (end 11.8502 4.826) (width 0.2) (layer "F.Cu") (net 1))
 (segment (start 8.626 23.3915) (end 9.698 23.3915) (width 0.2) (layer "F.Cu") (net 1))
 (segment (start 9.698 23.3915) (end 9.698 17.449) (width 0.2) (layer "F.Cu") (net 1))
 (segment (start 4.809 4.176) (end 3.698 4.176) (width 0.2) (layer "F.Cu") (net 1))
 (segment (start 11.8502 4.826) (end 11.938 4.9138) (width 0.2) (layer "F.Cu") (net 1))
 (segment (start 9.398 14.762) (end 10.558 14.762) (width 0.2) (layer "F.Cu") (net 1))
 (segment (start 8.89 15.27) (end 9.398 14.762) (width 0.2) (layer "F.Cu") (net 1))
 (segment (start 4.682 9.9124) (end 5.2219 9.3725) (width 0.2) (layer "F.Cu") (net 1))
 (segment (start 4.682 9.9124) (end 4.682 11.512) (width 0.2) (layer "F.Cu") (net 1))
 (segment (start 12.573 13.97) (end 12.573 5.5488) (width 0.2) (layer "F.Cu") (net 1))
 (segment (start 3.698 4.176) (end 3.302 4.572) (width 0.2) (layer "F.Cu") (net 1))
 (segment (start 8.89 16.641) (end 8.89 15.27) (width 0.2) (layer "F.Cu") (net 1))
 (segment (start 9.698 23.3915) (end 10.7735 23.3915) (width 0.2) (layer "F.Cu") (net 1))
 (segment (start 2.794 5.08) (end 3.302 4.572) (width 0.2) (layer "F.Cu") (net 1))
 (segment (start 2.794 8.7484) (end 2.794 5.08) (width 0.2) (layer "F.Cu") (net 1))
 (segment (start 9.698 17.449) (end 8.89 16.641) (width 0.2) (layer "F.Cu") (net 1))
 (segment (start 12.573 5.5488) (end 11.938 4.9138) (width 0.2) (layer "F.Cu") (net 1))
 (segment (start 11.781 14.762) (end 12.573 13.97) (width 0.2) (layer "F.Cu") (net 1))
 (via (at 5.2219 9.3725) (size 0.8) (drill 0.4) (layers "F.Cu" "B.Cu") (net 1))
 (via (at 2.794 8.7484) (size 0.8) (drill 0.4) (layers "F.Cu" "B.Cu") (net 1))
 (via (at 11.938 4.9138) (size 0.8) (drill 0.4) (layers "F.Cu" "B.Cu") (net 1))
 (via (at 3.302 4.572) (size 0.8) (drill 0.4) (layers "F.Cu" "B.Cu") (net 1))
 (segment (start 3.6438 4.9138) (end 11.938 4.9138) (width 0.2) (layer "B.Cu") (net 1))
 (segment (start 5.2219 9.3725) (end 4.5978 8.7484) (width 0.2) (layer "B.Cu") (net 1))
 (segment (start 4.5978 8.7484) (end 2.794 8.7484) (width 0.2) (layer "B.Cu") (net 1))
 (segment (start 3.302 4.572) (end 3.6438 4.9138) (width 0.2) (layer "B.Cu") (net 1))
 (segment (start 11.6225 6.126) (end 11.938 6.4415) (width 0.2) (layer "F.Cu") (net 27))
 (segment (start 11.938 6.4415) (end 11.938 13.7712) (width 0.2) (layer "F.Cu") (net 27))
 (segment (start 11.5972 14.112) (end 10.558 14.112) (width 0.2) (layer "F.Cu") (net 27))
 (segment (start 10.685 6.126) (end 11.6225 6.126) (width 0.2) (layer "F.Cu") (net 27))
 (segment (start 11.938 13.7712) (end 11.5972 14.112) (width 0.2) (layer "F.Cu") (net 27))
 (segment (start 4.682 12.162) (end 3.6428 12.162) (width 0.2) (layer "F.Cu") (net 25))
 (segment (start 3.6428 5.603) (end 3.7698 5.476) (width 0.2) (layer "F.Cu") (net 25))
 (segment (start 3.6428 12.162) (end 3.6428 5.603) (width 0.2) (layer "F.Cu") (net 25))
 (segment (start 4.809 5.476) (end 3.7698 5.476) (width 0.2) (layer "F.Cu") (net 25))
 (segment (start 6.457 21.905) (end 8.2875 21.905) (width 0.2) (layer "F.Cu") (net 2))
 (segment (start 12.5494 15.0163) (end 13.335 14.2307) (width 0.2) (layer "F.Cu") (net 13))
 (segment (start 13.335 14.2307) (end 13.335 4.826) (width 0.2) (layer "F.Cu") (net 13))
 (segment (start 12.685 4.176) (end 10.685 4.176) (width 0.2) (layer "F.Cu") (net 13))
 (segment (start 13.335 4.826) (end 12.685 4.176) (width 0.2) (layer "F.Cu") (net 13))
 (via (at 12.5494 15.0163) (size 0.8) (drill 0.4) (layers "F.Cu" "B.Cu") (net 13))
 (segment (start 4.7057 22.86) (end 12.5494 15.0163) (width 0.2) (layer "B.Cu") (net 13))
 (segment (start 0 22.86) (end 4.7057 22.86) (width 0.2) (layer "B.Cu") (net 13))
 (segment (start 2.938939 3.526) (end 2.032 4.432939) (width 0.2) (layer "F.Cu") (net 12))
 (segment (start 1.905 9.836) (end 1.905 15.875) (width 0.2) (layer "F.Cu") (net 12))
 (segment (start 2.032 4.432939) (end 2.032 9.709) (width 0.2) (layer "F.Cu") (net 12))
 (segment (start 2.032 9.709) (end 1.905 9.836) (width 0.2) (layer "F.Cu") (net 12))
 (segment (start 4.809 3.526) (end 2.938939 3.526) (width 0.2) (layer "F.Cu") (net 12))
 (segment (start 1.905 15.875) (end 0 17.78) (width 0.2) (layer "F.Cu") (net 12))
 (segment (start 2.204 2.876) (end 0 5.08) (width 0.2) (layer "F.Cu") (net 9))
 (segment (start 4.809 2.876) (end 2.204 2.876) (width 0.2) (layer "F.Cu") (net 9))
 (segment (start 11.968 3.526) (end 12.192 3.302) (width 0.2) (layer "F.Cu") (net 9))
 (segment (start 10.685 3.526) (end 11.968 3.526) (width 0.2) (layer "F.Cu") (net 9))
 (via (at 12.192 3.302) (size 0.8) (drill 0.4) (layers "F.Cu" "B.Cu") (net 9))
 (segment (start 0 5.08) (end 1.778 3.302) (width 0.2) (layer "B.Cu") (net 9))
 (segment (start 1.778 3.302) (end 12.192 3.302) (width 0.2) (layer "B.Cu") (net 9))
 (segment (start 3.4953 12.812) (end 2.657 13.6503) (width 0.2) (layer "F.Cu") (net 21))
 (segment (start 4.682 12.812) (end 3.4953 12.812) (width 0.2) (layer "F.Cu") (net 21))
 (segment (start 2.657 13.6503) (end 2.657 14.639) (width 0.2) (layer "F.Cu") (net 21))
 (via (at 2.657 14.639) (size 0.8) (drill 0.4) (layers "F.Cu" "B.Cu") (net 21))
 (segment (start 2.657 14.639) (end 9.6593 14.639) (width 0.2) (layer "B.Cu") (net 21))
 (segment (start 9.6593 14.639) (end 14.1383 10.16) (width 0.2) (layer "B.Cu") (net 21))
 (segment (start 15.24 10.16) (end 14.1383 10.16) (width 0.2) (layer "B.Cu") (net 21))
 (segment (start 15.24 17.78) (end 14.1383 17.78) (width 0.2) (layer "F.Cu") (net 18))
 (segment (start 10.558 15.412) (end 11.7703 15.412) (width 0.2) (layer "F.Cu") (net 18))
 (segment (start 11.7703 15.412) (end 14.1383 17.78) (width 0.2) (layer "F.Cu") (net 18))
 (segment (start 3.0276 20.955) (end 3.957 20.955) (width 0.2) (layer "F.Cu") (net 6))
 (segment (start 2.6252 20.5526) (end 3.0276 20.955) (width 0.2) (layer "F.Cu") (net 6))
 (via (at 2.6252 20.5526) (size 0.8) (drill 0.4) (layers "F.Cu" "B.Cu") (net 6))
 (segment (start 1.524 19.4514) (end 2.6252 20.5526) (width 0.2) (layer "B.Cu") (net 6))
 (segment (start 1.524 11.684) (end 1.524 19.4514) (width 0.2) (layer "B.Cu") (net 6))
 (segment (start 0 10.16) (end 1.524 11.684) (width 0.2) (layer "B.Cu") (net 6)))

